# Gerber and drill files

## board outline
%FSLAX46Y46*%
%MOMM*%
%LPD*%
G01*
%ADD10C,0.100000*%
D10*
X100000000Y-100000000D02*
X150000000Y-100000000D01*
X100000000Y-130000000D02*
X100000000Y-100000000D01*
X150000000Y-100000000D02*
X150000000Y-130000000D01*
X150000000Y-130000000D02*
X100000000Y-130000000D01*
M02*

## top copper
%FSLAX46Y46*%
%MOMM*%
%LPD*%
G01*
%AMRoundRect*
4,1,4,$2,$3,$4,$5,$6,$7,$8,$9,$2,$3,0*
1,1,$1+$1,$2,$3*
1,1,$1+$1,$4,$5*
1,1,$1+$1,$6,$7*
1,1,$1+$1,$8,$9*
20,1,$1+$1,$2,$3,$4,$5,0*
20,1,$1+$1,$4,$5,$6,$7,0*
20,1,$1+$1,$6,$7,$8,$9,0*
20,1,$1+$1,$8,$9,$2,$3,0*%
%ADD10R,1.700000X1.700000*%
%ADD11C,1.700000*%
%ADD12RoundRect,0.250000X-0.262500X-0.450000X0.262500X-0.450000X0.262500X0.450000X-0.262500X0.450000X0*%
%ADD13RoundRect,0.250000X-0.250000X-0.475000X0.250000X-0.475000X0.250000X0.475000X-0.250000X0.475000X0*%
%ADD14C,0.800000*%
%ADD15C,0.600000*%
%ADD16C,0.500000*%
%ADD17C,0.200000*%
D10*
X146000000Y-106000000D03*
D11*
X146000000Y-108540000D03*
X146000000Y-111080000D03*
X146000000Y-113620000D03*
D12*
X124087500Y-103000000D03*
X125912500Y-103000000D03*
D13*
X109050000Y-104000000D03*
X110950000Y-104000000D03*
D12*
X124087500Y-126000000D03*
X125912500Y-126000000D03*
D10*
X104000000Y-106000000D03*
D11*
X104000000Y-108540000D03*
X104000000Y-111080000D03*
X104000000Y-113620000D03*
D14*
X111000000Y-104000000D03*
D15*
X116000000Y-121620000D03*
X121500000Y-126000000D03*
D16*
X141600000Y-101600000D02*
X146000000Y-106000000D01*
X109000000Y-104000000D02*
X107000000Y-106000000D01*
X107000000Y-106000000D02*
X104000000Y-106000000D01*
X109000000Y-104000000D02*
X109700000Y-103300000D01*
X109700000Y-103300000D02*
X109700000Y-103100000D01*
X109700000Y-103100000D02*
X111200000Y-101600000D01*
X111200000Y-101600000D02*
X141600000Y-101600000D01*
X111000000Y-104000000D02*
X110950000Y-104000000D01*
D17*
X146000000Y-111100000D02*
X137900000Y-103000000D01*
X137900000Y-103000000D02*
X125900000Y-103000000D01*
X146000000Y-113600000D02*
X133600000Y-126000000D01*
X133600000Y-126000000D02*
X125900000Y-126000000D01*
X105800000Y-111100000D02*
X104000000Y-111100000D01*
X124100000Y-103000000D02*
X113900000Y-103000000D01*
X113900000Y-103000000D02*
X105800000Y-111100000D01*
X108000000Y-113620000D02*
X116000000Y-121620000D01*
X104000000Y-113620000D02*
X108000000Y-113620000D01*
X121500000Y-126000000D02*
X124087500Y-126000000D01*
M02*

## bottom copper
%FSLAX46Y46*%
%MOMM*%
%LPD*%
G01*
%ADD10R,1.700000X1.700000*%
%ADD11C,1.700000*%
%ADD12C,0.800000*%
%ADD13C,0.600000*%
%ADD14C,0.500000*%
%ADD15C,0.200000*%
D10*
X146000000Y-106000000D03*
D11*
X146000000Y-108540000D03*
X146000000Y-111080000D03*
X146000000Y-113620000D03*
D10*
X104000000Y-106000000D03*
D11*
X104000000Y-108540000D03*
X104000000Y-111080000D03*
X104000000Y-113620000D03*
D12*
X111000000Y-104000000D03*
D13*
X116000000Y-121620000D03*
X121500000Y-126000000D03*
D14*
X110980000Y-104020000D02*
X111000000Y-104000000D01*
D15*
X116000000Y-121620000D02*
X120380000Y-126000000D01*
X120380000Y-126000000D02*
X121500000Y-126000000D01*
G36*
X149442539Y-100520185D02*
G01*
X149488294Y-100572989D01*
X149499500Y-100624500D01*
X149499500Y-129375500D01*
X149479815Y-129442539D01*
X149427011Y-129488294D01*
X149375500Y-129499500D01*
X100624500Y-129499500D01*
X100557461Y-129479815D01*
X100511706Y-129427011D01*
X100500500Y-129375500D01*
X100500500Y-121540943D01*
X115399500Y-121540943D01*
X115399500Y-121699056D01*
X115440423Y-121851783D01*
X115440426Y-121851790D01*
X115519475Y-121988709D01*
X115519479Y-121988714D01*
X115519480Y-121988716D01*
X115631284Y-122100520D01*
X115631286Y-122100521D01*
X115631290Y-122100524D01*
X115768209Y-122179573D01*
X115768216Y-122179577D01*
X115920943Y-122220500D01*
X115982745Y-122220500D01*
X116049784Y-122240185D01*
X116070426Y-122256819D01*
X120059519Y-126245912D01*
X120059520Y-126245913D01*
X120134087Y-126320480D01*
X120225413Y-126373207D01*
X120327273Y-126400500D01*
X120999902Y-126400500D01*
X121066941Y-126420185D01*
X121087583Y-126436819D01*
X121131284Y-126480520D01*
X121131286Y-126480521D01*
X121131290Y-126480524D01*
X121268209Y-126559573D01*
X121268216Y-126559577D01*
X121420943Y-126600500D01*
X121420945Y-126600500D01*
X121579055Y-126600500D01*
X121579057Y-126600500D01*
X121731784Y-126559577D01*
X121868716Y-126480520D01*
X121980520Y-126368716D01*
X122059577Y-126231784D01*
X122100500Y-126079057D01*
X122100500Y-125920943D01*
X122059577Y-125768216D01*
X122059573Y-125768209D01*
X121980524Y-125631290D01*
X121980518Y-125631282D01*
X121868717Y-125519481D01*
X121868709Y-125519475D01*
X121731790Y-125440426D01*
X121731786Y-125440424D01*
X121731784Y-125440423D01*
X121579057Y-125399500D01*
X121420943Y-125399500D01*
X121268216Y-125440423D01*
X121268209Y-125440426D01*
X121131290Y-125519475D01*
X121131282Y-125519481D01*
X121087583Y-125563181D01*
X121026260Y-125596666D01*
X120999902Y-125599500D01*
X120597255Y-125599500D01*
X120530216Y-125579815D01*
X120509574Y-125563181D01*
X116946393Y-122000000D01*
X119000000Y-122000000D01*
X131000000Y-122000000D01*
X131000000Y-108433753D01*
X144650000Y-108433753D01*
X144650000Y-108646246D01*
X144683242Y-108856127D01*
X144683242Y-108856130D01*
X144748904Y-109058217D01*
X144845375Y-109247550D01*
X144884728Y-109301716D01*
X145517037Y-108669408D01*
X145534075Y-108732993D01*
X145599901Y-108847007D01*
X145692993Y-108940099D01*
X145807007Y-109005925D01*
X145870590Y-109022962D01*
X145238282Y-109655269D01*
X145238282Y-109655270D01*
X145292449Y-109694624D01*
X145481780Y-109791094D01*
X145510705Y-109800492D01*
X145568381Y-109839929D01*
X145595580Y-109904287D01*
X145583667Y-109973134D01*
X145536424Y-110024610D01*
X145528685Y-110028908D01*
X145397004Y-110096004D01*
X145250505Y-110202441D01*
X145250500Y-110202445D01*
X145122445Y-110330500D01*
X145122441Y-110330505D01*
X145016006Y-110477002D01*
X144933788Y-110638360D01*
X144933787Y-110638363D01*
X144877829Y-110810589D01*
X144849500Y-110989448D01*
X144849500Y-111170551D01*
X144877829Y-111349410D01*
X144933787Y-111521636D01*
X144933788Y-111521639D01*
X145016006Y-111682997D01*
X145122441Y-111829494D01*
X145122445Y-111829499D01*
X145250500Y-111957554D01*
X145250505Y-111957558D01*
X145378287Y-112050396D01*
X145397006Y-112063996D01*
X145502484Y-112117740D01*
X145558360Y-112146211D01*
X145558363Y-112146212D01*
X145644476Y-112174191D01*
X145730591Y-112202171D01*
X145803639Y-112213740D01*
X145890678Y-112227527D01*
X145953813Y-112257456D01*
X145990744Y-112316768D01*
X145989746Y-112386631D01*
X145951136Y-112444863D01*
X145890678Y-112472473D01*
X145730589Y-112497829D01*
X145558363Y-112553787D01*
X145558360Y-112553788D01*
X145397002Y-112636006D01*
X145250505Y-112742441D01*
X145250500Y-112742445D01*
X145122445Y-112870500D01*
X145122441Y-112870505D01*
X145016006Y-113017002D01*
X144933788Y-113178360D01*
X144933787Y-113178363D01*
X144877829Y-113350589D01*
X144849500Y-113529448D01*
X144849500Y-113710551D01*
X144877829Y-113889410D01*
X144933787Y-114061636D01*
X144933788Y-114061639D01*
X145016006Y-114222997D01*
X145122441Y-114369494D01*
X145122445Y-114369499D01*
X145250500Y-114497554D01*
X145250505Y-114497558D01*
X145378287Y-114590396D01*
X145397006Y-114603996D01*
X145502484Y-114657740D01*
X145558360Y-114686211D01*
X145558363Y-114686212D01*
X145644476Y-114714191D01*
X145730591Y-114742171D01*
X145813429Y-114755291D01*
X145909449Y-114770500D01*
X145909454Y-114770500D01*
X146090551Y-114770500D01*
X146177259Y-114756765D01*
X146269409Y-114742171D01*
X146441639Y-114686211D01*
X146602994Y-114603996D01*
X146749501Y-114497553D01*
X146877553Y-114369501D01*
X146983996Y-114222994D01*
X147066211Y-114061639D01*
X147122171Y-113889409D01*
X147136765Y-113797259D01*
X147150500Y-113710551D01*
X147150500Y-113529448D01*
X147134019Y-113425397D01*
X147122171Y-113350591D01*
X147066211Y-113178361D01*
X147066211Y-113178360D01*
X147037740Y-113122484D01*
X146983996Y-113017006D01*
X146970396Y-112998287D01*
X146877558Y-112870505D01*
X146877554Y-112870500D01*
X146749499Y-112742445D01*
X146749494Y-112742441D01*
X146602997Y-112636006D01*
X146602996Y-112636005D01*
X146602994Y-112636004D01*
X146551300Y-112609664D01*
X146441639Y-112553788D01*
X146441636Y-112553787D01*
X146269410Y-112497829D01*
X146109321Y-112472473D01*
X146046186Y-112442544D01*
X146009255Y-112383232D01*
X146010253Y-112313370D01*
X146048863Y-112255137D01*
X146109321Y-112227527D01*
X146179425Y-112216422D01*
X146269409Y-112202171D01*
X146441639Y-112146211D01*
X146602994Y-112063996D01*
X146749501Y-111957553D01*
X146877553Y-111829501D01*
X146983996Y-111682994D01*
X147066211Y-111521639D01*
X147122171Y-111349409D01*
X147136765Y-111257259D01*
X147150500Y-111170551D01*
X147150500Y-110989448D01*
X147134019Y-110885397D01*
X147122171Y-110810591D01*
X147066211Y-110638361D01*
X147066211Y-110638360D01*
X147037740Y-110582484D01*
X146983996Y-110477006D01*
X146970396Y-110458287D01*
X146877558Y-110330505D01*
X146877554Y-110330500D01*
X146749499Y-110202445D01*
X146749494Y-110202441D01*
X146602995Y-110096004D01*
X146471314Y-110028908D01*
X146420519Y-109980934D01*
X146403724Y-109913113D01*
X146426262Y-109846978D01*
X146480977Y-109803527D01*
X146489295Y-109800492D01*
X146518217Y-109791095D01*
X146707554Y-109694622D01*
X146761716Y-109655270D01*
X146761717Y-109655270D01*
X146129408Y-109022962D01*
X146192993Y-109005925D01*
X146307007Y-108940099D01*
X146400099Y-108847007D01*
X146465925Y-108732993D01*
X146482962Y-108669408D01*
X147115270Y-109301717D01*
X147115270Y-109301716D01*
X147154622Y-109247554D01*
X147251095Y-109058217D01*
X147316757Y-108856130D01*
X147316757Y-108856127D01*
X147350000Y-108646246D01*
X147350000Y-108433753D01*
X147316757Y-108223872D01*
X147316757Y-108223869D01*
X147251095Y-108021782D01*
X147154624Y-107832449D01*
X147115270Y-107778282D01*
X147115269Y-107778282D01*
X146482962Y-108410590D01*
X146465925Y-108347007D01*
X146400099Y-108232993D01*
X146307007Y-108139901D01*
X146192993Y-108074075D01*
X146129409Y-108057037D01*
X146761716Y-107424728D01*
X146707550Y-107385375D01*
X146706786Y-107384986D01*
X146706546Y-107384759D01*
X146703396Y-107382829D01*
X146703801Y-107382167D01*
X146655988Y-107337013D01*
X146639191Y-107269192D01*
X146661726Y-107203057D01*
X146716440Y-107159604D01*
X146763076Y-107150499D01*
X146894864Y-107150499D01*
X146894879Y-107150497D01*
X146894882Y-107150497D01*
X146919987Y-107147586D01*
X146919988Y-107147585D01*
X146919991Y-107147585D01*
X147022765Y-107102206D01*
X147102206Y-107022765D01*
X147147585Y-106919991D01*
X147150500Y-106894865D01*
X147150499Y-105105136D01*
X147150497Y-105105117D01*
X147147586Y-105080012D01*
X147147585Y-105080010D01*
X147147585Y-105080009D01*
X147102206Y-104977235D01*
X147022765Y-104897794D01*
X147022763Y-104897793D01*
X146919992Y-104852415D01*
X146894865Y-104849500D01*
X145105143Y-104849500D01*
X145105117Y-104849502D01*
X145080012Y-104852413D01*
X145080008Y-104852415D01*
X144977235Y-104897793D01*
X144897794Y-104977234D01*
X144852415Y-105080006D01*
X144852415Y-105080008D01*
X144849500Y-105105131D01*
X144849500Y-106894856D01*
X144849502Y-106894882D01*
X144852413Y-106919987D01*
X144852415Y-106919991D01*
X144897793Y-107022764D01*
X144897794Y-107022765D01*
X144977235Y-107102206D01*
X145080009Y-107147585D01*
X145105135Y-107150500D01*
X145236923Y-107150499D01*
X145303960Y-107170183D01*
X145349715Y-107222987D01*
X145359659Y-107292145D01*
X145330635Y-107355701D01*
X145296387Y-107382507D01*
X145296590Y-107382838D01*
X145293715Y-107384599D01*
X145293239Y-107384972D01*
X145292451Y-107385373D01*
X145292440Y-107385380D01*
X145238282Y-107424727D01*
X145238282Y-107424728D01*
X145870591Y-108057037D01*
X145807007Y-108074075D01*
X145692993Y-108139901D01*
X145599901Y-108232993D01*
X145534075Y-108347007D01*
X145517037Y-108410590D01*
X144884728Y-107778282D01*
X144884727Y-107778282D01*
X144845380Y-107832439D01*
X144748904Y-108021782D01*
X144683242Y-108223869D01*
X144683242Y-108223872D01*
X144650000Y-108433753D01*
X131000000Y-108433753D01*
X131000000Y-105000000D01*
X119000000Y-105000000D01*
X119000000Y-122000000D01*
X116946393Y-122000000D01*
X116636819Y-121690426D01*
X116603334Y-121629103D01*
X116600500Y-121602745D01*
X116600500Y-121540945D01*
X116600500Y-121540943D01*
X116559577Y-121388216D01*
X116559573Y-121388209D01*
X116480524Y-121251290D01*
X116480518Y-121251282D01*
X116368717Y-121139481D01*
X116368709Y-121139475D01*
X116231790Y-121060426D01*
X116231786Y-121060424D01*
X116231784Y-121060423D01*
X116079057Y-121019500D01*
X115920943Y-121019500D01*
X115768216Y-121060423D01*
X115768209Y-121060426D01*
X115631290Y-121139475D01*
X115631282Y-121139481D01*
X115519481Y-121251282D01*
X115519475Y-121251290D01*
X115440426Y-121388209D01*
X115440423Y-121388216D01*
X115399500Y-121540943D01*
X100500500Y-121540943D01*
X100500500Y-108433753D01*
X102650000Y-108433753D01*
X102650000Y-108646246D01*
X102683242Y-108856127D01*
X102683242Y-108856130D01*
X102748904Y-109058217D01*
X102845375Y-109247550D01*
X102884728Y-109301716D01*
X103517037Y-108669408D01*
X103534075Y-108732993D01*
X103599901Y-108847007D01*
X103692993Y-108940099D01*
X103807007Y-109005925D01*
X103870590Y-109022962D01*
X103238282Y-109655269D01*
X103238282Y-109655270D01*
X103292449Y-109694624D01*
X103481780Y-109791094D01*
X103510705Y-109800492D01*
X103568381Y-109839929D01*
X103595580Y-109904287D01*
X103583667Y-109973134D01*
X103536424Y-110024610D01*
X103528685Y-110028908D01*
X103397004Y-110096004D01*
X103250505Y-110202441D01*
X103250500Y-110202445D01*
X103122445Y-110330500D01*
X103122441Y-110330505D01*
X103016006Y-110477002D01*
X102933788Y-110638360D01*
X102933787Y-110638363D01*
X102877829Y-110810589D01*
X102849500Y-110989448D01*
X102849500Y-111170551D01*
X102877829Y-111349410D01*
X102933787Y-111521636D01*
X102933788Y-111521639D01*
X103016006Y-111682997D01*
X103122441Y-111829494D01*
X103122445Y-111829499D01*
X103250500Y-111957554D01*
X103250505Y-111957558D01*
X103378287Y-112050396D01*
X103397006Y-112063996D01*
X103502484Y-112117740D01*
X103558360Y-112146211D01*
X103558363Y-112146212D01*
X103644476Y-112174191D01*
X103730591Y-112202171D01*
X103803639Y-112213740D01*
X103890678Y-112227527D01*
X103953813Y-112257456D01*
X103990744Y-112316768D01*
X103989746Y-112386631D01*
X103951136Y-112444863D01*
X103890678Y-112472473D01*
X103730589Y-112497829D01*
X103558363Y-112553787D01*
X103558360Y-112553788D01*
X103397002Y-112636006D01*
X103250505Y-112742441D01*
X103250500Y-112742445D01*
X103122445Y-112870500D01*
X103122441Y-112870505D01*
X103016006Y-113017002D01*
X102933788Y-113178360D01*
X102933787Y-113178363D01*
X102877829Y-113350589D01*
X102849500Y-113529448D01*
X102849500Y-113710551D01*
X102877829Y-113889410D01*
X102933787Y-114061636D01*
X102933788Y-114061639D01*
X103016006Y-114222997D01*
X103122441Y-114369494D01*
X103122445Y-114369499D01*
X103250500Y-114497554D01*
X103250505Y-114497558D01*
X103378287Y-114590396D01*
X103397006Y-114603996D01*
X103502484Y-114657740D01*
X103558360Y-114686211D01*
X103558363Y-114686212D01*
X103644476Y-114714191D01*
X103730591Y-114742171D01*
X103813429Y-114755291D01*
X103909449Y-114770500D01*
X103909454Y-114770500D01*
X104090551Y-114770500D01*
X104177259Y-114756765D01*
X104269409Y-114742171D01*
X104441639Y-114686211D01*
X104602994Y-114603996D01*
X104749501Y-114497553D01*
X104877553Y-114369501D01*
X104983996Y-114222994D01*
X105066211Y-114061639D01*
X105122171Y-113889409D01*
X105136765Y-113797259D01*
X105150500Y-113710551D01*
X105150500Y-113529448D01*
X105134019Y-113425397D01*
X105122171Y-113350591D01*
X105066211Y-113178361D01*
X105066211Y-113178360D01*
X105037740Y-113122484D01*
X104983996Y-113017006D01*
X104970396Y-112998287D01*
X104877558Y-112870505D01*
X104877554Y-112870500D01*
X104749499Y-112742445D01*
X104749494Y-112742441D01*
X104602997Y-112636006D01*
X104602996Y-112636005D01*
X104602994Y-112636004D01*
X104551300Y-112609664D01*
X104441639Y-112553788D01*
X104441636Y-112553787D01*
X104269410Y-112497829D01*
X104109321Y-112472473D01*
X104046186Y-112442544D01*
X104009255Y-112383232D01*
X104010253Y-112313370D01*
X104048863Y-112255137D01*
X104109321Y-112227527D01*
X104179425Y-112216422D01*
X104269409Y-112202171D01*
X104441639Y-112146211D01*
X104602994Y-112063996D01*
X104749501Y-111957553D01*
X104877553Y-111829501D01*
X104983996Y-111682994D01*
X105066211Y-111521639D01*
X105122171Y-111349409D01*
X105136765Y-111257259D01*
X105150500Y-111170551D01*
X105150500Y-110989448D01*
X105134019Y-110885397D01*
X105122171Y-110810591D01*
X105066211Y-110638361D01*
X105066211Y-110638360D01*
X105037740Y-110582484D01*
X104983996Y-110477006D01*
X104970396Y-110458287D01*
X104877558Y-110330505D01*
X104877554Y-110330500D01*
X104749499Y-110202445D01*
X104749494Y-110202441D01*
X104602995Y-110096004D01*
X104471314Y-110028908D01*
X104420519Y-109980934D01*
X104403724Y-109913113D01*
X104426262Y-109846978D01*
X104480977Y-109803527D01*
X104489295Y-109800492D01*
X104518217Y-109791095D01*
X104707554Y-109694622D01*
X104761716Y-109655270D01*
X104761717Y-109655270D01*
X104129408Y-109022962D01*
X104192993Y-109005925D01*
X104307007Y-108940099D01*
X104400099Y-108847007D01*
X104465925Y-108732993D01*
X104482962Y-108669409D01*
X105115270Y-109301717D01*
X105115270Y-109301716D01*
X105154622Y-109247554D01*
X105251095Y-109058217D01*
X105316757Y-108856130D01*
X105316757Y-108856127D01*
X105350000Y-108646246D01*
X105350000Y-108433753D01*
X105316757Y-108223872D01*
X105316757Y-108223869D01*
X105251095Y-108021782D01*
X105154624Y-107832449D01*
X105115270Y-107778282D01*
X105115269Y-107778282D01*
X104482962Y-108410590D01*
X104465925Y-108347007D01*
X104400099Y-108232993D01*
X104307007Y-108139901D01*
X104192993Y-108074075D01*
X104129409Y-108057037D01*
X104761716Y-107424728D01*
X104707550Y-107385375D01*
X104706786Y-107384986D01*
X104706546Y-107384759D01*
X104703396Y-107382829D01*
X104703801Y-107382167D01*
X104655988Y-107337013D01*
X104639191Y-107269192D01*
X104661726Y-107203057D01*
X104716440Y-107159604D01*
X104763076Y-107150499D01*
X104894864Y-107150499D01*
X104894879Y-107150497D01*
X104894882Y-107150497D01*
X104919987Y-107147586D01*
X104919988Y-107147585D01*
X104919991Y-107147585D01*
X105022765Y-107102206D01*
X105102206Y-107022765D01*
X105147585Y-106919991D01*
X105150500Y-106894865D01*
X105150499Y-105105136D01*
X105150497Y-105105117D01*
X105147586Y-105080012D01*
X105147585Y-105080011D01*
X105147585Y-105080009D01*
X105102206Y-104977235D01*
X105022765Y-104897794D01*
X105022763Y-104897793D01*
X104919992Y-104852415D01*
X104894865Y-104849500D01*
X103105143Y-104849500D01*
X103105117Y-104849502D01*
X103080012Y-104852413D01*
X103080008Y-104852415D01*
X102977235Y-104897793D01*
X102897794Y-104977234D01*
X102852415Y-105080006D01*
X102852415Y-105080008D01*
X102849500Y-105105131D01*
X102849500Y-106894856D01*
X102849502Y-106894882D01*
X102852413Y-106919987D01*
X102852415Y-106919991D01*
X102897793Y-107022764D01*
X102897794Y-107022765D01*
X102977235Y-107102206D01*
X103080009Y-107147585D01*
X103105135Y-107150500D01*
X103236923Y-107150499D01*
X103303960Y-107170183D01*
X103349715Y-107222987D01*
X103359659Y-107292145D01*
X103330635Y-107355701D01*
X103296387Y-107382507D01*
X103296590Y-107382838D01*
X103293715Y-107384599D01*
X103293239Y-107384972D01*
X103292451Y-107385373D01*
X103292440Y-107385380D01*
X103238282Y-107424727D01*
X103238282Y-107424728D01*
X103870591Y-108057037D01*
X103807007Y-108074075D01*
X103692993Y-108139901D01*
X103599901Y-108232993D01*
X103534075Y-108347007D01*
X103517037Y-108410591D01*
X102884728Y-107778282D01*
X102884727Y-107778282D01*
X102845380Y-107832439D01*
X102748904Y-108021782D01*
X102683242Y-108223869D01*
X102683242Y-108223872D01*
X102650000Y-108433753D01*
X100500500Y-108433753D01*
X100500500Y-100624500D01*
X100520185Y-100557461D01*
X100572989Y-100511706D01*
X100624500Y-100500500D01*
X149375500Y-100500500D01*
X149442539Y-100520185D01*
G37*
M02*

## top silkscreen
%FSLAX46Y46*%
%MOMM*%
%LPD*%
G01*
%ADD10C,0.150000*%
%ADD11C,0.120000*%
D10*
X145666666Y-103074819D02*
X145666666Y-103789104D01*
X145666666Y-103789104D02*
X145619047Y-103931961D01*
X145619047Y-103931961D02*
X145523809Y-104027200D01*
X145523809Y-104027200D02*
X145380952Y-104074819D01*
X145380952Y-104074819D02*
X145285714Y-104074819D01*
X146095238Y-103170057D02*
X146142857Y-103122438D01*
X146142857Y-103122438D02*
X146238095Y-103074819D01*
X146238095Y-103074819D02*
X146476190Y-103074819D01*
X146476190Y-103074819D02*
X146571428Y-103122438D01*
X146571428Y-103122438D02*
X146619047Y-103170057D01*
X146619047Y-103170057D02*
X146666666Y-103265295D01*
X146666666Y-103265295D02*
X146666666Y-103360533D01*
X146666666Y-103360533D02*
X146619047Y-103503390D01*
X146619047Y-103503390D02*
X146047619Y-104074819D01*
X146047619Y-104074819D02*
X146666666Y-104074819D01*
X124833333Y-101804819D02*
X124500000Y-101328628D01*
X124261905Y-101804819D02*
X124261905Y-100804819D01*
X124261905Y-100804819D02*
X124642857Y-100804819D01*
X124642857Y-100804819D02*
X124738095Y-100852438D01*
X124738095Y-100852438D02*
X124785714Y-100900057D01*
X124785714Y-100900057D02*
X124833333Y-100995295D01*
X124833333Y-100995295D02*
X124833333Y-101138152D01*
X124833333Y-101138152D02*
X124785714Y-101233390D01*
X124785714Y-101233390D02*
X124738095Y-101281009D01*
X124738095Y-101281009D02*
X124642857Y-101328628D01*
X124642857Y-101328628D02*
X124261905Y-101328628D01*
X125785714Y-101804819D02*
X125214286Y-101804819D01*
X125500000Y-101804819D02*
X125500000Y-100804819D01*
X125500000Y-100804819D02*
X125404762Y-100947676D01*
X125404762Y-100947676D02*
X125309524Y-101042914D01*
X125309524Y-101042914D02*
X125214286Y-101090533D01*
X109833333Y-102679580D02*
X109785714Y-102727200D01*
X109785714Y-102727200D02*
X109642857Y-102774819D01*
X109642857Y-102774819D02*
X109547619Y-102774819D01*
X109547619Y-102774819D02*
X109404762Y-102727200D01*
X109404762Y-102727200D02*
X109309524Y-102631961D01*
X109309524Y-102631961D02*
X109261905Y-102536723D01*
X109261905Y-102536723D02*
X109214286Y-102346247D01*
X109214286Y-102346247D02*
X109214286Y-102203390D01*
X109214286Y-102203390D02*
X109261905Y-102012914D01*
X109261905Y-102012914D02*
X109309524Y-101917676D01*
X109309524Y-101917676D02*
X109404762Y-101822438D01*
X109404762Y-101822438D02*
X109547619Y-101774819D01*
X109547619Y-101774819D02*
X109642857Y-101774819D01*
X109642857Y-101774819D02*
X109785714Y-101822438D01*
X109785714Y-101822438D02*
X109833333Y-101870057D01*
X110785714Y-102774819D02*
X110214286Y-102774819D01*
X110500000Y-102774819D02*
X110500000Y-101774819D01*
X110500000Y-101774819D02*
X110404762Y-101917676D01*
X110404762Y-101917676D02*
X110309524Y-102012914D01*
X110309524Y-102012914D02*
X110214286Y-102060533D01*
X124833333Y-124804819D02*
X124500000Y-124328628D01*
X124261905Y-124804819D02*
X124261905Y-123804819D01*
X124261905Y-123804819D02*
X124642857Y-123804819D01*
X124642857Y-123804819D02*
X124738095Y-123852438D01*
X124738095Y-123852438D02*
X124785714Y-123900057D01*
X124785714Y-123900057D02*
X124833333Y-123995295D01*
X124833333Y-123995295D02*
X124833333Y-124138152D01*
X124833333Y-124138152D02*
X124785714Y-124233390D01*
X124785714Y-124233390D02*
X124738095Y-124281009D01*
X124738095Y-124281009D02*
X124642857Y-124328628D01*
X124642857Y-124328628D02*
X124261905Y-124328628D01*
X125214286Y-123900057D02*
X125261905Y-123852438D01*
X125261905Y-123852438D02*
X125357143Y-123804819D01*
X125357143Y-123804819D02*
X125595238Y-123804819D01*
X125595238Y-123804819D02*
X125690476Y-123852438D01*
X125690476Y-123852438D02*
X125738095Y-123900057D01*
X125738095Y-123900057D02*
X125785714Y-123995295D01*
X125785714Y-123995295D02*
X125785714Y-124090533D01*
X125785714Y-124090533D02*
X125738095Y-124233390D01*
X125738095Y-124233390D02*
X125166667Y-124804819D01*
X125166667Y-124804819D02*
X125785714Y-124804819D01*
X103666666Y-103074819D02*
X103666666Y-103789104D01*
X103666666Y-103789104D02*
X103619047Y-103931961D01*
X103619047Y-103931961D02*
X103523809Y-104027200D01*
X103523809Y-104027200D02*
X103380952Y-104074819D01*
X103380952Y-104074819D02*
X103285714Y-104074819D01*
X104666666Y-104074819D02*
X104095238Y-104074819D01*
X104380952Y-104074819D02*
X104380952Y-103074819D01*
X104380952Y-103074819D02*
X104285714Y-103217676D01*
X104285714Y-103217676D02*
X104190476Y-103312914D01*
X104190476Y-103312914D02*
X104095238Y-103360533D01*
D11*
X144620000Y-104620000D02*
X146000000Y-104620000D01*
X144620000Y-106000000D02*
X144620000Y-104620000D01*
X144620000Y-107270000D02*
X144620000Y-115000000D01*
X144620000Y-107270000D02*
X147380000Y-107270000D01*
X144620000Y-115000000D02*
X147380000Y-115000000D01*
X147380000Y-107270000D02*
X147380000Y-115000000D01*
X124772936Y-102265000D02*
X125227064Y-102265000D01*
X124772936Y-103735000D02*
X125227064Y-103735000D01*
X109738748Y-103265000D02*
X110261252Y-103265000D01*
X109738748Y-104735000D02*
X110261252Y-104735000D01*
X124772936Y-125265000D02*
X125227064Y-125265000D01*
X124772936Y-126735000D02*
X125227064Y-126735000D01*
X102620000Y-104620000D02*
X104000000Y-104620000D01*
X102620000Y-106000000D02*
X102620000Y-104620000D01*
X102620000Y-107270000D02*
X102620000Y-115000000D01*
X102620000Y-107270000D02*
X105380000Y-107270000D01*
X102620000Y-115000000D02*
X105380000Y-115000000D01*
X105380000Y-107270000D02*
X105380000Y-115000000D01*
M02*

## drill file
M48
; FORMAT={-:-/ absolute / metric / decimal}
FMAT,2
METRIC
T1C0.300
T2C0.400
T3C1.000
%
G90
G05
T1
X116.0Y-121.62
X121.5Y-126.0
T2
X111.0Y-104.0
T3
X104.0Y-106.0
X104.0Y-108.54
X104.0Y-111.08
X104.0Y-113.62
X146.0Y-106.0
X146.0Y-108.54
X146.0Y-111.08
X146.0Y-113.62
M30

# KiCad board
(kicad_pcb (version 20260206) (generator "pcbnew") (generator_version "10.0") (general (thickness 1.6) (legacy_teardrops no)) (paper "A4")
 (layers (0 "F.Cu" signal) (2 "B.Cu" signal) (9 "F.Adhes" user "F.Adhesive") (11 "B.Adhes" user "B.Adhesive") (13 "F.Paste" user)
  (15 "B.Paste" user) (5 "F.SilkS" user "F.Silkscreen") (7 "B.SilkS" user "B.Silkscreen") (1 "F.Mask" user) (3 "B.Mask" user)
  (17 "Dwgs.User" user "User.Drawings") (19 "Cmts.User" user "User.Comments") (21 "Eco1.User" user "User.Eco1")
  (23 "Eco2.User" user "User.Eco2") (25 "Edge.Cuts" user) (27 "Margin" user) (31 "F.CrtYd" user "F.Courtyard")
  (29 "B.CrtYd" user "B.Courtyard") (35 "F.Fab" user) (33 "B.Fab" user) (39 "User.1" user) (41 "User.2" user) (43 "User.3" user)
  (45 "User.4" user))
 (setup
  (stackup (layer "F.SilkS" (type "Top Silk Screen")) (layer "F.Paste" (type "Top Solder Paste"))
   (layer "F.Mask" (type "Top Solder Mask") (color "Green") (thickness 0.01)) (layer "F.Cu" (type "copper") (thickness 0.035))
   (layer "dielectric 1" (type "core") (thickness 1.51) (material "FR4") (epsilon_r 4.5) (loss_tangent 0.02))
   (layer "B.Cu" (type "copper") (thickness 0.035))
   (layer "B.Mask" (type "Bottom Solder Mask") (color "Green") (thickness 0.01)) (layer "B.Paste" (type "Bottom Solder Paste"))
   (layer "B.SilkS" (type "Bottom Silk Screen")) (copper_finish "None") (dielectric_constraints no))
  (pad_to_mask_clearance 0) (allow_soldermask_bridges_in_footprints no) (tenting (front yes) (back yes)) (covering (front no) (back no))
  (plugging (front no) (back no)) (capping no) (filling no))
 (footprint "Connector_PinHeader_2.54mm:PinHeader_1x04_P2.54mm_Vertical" (layer "F.Cu") (at 146 106)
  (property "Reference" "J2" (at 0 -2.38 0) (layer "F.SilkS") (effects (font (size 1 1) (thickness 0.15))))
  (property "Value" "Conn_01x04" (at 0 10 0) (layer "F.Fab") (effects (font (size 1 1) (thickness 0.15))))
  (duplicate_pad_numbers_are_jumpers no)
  (fp_line (start -1.38 -1.38) (end 0 -1.38) (stroke (width 0.12) (type solid)) (layer "F.SilkS"))
  (fp_line (start -1.38 0) (end -1.38 -1.38) (stroke (width 0.12) (type solid)) (layer "F.SilkS"))
  (fp_line (start -1.38 1.27) (end -1.38 9) (stroke (width 0.12) (type solid)) (layer "F.SilkS"))
  (fp_line (start -1.38 1.27) (end 1.38 1.27) (stroke (width 0.12) (type solid)) (layer "F.SilkS"))
  (fp_line (start -1.38 9) (end 1.38 9) (stroke (width 0.12) (type solid)) (layer "F.SilkS"))
  (fp_line (start 1.38 1.27) (end 1.38 9) (stroke (width 0.12) (type solid)) (layer "F.SilkS"))
  (pad "1" thru_hole rect (at 0 0) (size 1.7 1.7) (drill 1) (layers "*.Cu" "*.Mask") (remove_unused_layers no) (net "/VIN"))
  (pad "2" thru_hole circle (at 0 2.54) (size 1.7 1.7) (drill 1) (layers "*.Cu" "*.Mask") (remove_unused_layers no) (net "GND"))
  (pad "3" thru_hole circle (at 0 5.08) (size 1.7 1.7) (drill 1) (layers "*.Cu" "*.Mask") (remove_unused_layers no) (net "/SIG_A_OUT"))
  (pad "4" thru_hole circle (at 0 7.62) (size 1.7 1.7) (drill 1) (layers "*.Cu" "*.Mask") (remove_unused_layers no) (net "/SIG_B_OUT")))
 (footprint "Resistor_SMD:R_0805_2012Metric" (layer "F.Cu") (at 125 103)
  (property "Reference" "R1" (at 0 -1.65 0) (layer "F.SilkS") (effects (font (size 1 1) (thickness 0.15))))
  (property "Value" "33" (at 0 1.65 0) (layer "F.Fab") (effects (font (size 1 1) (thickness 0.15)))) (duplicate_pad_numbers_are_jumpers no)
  (fp_line (start -0.227064 -0.735) (end 0.227064 -0.735) (stroke (width 0.12) (type solid)) (layer "F.SilkS"))
  (fp_line (start -0.227064 0.735) (end 0.227064 0.735) (stroke (width 0.12) (type solid)) (layer "F.SilkS"))
  (pad "1" smd roundrect (at -0.9125 0) (size 1.025 1.4) (layers "F.Cu" "F.Mask" "F.Paste") (roundrect_rratio 0.243902) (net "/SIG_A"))
  (pad "2" smd roundrect (at 0.9125 0) (size 1.025 1.4) (layers "F.Cu" "F.Mask" "F.Paste") (roundrect_rratio 0.243902) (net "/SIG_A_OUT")))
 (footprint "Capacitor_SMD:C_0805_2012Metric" (layer "F.Cu") (at 110 104)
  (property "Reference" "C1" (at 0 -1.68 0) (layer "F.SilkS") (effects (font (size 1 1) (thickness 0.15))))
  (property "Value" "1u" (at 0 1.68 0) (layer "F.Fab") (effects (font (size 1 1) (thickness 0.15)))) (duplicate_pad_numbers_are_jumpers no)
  (fp_line (start -0.261252 -0.735) (end 0.261252 -0.735) (stroke (width 0.12) (type solid)) (layer "F.SilkS"))
  (fp_line (start -0.261252 0.735) (end 0.261252 0.735) (stroke (width 0.12) (type solid)) (layer "F.SilkS"))
  (pad "1" smd roundrect (at -0.95 0) (size 1 1.45) (layers "F.Cu" "F.Mask" "F.Paste") (roundrect_rratio 0.25) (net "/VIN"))
  (pad "2" smd roundrect (at 0.95 0) (size 1 1.45) (layers "F.Cu" "F.Mask" "F.Paste") (roundrect_rratio 0.25) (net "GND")))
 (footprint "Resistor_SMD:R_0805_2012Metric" (layer "F.Cu") (at 125 126)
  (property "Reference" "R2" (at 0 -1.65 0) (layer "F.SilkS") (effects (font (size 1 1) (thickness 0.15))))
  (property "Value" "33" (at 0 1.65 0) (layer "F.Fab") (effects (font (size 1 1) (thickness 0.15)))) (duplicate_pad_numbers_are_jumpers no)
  (fp_line (start -0.227064 -0.735) (end 0.227064 -0.735) (stroke (width 0.12) (type solid)) (layer "F.SilkS"))
  (fp_line (start -0.227064 0.735) (end 0.227064 0.735) (stroke (width 0.12) (type solid)) (layer "F.SilkS"))
  (pad "1" smd roundrect (at -0.9125 0) (size 1.025 1.4) (layers "F.Cu" "F.Mask" "F.Paste") (roundrect_rratio 0.243902) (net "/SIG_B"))
  (pad "2" smd roundrect (at 0.9125 0) (size 1.025 1.4) (layers "F.Cu" "F.Mask" "F.Paste") (roundrect_rratio 0.243902) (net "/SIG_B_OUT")))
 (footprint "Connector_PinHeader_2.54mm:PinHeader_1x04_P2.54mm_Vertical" (layer "F.Cu") (at 104 106)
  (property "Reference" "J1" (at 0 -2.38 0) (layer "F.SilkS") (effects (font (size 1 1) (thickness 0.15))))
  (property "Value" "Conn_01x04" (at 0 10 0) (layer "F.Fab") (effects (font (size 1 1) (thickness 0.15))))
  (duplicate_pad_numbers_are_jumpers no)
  (fp_line (start -1.38 -1.38) (end 0 -1.38) (stroke (width 0.12) (type solid)) (layer "F.SilkS"))
  (fp_line (start -1.38 0) (end -1.38 -1.38) (stroke (width 0.12) (type solid)) (layer "F.SilkS"))
  (fp_line (start -1.38 1.27) (end -1.38 9) (stroke (width 0.12) (type solid)) (layer "F.SilkS"))
  (fp_line (start -1.38 1.27) (end 1.38 1.27) (stroke (width 0.12) (type solid)) (layer "F.SilkS"))
  (fp_line (start -1.38 9) (end 1.38 9) (stroke (width 0.12) (type solid)) (layer "F.SilkS"))
  (fp_line (start 1.38 1.27) (end 1.38 9) (stroke (width 0.12) (type solid)) (layer "F.SilkS"))
  (pad "1" thru_hole rect (at 0 0) (size 1.7 1.7) (drill 1) (layers "*.Cu" "*.Mask") (remove_unused_layers no) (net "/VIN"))
  (pad "2" thru_hole circle (at 0 2.54) (size 1.7 1.7) (drill 1) (layers "*.Cu" "*.Mask") (remove_unused_layers no) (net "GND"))
  (pad "3" thru_hole circle (at 0 5.08) (size 1.7 1.7) (drill 1) (layers "*.Cu" "*.Mask") (remove_unused_layers no) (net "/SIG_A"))
  (pad "4" thru_hole circle (at 0 7.62) (size 1.7 1.7) (drill 1) (layers "*.Cu" "*.Mask") (remove_unused_layers no) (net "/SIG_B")))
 (gr_line (start 100 100) (end 150 100) (stroke (width 0.1) (type default)) (layer "Edge.Cuts"))
 (gr_line (start 100 130) (end 100 100) (stroke (width 0.1) (type default)) (layer "Edge.Cuts"))
 (gr_line (start 150 100) (end 150 130) (stroke (width 0.1) (type default)) (layer "Edge.Cuts"))
 (gr_line (start 150 130) (end 100 130) (stroke (width 0.1) (type default)) (layer "Edge.Cuts"))
 (segment (start 141.6 101.6) (end 146 106) (width 0.5) (layer "F.Cu") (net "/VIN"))
 (segment (start 109 104) (end 107 106) (width 0.5) (layer "F.Cu") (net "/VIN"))
 (segment (start 107 106) (end 104 106) (width 0.5) (layer "F.Cu") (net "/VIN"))
 (segment (start 109 104) (end 109.7 103.3) (width 0.5) (layer "F.Cu") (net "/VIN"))
 (segment (start 109.7 103.3) (end 109.7 103.1) (width 0.5) (layer "F.Cu") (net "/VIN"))
 (segment (start 109.7 103.1) (end 111.2 101.6) (width 0.5) (layer "F.Cu") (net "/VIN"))
 (segment (start 111.2 101.6) (end 141.6 101.6) (width 0.5) (layer "F.Cu") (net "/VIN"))
 (segment (start 111 104) (end 110.95 104) (width 0.5) (layer "F.Cu") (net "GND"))
 (via (at 111 104) (size 0.8) (drill 0.4) (layers "F.Cu" "B.Cu") (capping yes) (filling yes) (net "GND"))
 (segment (start 110.98 104.02) (end 111 104) (width 0.5) (layer "B.Cu") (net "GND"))
 (segment (start 146 111.1) (end 137.9 103) (width 0.2) (layer "F.Cu") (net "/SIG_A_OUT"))
 (segment (start 137.9 103) (end 125.9 103) (width 0.2) (layer "F.Cu") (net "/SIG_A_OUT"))
 (segment (start 146 113.6) (end 133.6 126) (width 0.2) (layer "F.Cu") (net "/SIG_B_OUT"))
 (segment (start 133.6 126) (end 125.9 126) (width 0.2) (layer "F.Cu") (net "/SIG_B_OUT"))
 (segment (start 105.8 111.1) (end 104 111.1) (width 0.2) (layer "F.Cu") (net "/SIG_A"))
 (segment (start 124.1 103) (end 113.9 103) (width 0.2) (layer "F.Cu") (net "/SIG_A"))
 (segment (start 113.9 103) (end 105.8 111.1) (width 0.2) (layer "F.Cu") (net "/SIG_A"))
 (segment (start 108 113.62) (end 116 121.62) (width 0.2) (locked yes) (layer "F.Cu") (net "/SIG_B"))
 (segment (start 104 113.62) (end 108 113.62) (width 0.2) (locked yes) (layer "F.Cu") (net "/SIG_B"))
 (segment (start 121.5 126) (end 124.0875 126) (width 0.2) (locked yes) (layer "F.Cu") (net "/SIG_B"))
 (via (at 116 121.62) (size 0.6) (drill 0.3) (layers "F.Cu" "B.Cu") (locked yes) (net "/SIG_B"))
 (via (at 121.5 126) (size 0.6) (drill 0.3) (layers "F.Cu" "B.Cu") (locked yes) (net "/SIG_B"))
 (segment (start 116 121.62) (end 120.38 126) (width 0.2) (locked yes) (layer "B.Cu") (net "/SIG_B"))
 (segment (start 120.38 126) (end 121.5 126) (width 0.2) (locked yes) (layer "B.Cu") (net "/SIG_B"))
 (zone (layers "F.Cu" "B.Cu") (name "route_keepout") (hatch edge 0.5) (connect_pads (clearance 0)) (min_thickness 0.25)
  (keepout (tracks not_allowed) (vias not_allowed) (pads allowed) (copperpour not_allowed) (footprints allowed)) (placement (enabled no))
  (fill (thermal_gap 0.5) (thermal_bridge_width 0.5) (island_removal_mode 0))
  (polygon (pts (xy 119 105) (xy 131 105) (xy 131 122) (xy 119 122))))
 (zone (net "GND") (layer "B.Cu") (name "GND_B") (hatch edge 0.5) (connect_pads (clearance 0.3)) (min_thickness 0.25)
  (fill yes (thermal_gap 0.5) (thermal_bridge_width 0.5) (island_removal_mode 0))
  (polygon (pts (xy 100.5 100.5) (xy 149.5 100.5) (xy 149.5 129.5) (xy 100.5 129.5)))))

